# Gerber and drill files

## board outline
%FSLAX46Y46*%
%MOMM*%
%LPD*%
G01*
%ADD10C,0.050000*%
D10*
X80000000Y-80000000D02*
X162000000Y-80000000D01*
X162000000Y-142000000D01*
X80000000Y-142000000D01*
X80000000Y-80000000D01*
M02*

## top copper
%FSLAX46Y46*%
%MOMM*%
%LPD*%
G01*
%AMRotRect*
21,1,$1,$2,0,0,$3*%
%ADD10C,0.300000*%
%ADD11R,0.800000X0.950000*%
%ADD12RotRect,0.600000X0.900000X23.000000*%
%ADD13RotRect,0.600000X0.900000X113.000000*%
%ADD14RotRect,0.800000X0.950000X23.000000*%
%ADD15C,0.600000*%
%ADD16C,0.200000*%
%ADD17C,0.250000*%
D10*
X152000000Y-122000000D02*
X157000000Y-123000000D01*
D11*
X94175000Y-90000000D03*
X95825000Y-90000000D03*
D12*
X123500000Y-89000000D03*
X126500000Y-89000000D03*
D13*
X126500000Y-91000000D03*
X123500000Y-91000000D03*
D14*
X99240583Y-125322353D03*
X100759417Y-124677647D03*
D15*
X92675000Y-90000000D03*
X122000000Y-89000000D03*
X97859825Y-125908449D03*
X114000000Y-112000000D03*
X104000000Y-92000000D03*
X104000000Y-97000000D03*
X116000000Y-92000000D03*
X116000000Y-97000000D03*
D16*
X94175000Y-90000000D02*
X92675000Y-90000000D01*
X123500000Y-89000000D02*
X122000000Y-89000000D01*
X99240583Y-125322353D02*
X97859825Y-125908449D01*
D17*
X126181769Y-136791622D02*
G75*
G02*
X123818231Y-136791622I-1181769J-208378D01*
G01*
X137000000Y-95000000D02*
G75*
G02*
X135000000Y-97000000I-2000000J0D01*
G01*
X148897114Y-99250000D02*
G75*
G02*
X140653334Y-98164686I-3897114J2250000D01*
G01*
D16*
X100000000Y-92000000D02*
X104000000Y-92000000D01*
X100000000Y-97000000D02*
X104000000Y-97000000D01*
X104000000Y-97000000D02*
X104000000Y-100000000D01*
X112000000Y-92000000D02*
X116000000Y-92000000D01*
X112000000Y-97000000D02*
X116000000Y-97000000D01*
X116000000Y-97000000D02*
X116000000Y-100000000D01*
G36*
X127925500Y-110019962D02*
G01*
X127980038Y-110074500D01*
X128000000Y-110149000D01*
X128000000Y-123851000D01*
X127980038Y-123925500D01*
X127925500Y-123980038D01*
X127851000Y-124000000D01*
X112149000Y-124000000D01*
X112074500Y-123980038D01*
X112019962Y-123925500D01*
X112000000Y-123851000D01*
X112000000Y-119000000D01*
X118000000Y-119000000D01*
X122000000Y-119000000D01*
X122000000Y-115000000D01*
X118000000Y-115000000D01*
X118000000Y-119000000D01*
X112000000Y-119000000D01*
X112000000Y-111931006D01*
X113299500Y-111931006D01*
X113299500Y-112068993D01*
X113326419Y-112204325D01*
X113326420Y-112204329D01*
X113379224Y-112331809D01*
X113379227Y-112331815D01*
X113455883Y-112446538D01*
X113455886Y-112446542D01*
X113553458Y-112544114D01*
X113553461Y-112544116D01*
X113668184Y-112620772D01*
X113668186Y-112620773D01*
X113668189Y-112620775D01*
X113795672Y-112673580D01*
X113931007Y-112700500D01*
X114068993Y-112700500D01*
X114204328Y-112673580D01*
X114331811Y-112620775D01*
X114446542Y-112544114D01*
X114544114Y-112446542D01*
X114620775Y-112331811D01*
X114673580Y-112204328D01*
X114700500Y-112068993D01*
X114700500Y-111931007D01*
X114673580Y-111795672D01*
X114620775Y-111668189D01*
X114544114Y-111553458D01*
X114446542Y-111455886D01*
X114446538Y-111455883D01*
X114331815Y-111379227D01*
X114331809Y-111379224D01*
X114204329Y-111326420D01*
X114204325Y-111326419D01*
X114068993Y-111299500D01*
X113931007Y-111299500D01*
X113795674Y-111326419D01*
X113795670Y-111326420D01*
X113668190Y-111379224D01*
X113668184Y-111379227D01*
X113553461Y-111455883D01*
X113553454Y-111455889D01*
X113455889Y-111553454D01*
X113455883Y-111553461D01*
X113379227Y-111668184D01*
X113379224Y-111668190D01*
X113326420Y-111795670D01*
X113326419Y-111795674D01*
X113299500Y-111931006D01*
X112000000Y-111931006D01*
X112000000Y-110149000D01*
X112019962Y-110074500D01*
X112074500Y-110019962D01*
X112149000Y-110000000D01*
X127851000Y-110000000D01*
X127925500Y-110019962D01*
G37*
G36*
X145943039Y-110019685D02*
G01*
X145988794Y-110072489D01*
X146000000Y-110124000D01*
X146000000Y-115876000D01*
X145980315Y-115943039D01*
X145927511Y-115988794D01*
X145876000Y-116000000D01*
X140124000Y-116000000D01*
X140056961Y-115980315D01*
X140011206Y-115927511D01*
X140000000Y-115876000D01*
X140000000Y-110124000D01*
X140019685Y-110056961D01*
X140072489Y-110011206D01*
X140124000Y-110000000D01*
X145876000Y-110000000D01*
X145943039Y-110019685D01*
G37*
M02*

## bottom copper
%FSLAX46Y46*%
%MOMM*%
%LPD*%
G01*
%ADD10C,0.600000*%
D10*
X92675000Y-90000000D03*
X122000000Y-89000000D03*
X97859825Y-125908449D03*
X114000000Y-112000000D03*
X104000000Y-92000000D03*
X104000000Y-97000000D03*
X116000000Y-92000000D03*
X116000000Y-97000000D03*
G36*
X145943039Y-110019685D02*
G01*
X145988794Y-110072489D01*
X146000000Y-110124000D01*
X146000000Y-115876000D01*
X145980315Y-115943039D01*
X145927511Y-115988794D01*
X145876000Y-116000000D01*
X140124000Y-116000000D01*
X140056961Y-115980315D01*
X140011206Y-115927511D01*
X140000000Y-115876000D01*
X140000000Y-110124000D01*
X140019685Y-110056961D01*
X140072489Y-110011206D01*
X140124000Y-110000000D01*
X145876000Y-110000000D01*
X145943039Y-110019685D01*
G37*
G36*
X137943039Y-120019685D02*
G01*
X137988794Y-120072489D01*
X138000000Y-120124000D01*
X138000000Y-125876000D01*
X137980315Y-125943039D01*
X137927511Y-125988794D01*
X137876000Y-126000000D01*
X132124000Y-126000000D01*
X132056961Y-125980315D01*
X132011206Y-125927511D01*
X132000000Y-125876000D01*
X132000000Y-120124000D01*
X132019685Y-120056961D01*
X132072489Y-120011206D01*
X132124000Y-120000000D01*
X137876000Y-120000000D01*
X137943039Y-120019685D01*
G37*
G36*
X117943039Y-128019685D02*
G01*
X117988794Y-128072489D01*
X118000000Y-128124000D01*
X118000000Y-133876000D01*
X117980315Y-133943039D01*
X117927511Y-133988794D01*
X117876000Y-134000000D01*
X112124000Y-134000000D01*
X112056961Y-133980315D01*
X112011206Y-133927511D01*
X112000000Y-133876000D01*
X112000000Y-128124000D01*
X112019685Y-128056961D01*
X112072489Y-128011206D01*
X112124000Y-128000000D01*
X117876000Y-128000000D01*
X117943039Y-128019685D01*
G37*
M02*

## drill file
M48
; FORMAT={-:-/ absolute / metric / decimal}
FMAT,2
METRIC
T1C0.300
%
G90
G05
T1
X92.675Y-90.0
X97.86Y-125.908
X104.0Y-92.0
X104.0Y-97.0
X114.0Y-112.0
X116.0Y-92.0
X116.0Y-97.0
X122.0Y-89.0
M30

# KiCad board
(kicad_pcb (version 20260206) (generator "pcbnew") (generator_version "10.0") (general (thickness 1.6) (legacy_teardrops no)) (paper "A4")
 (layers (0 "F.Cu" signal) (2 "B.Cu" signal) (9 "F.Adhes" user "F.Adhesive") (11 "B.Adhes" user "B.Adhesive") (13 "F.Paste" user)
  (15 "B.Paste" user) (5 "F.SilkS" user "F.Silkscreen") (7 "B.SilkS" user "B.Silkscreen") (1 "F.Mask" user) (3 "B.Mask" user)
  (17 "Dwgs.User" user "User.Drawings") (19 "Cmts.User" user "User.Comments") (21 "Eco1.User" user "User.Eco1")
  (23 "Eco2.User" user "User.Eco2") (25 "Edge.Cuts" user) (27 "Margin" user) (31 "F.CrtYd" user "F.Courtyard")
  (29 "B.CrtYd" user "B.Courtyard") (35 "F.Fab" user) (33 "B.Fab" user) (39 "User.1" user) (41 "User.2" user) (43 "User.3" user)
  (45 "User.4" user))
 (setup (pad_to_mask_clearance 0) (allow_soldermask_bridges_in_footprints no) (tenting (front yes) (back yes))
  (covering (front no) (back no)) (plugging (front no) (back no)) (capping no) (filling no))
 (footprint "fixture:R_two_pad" (layer "F.Cu") (at 95 90)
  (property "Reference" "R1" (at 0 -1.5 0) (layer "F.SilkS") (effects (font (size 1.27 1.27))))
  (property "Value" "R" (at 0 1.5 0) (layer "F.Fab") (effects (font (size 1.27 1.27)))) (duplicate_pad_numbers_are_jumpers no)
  (pad "1" smd rect (at -0.825 0) (size 0.8 0.95) (layers "F.Cu" "F.Mask" "F.Paste") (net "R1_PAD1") (thermal_bridge_angle 45))
  (pad "2" smd rect (at 0.825 0) (size 0.8 0.95) (layers "F.Cu" "F.Mask" "F.Paste") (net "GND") (thermal_bridge_angle 45)))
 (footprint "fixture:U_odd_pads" (layer "F.Cu") (at 125 90)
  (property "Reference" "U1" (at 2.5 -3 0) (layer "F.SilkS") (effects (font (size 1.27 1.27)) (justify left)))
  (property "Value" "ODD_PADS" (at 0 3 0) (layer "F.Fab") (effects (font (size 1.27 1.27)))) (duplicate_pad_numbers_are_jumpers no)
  (pad "1" smd rect (at -1.5 -1 23) (size 0.6 0.9) (layers "F.Cu" "F.Mask" "F.Paste") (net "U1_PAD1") (thermal_bridge_angle 45))
  (pad "2" smd rect (at 1.5 -1 23) (size 0.6 0.9) (layers "F.Cu" "F.Mask" "F.Paste") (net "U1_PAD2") (thermal_bridge_angle 45))
  (pad "3" smd rect (at 1.5 1 113) (size 0.6 0.9) (layers "F.Cu" "F.Mask" "F.Paste") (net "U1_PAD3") (thermal_bridge_angle 45))
  (pad "4" smd rect (at -1.5 1 113) (size 0.6 0.9) (layers "F.Cu" "F.Mask" "F.Paste") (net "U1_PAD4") (thermal_bridge_angle 45)))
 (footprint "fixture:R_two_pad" (layer "F.Cu") (at 100 125 23)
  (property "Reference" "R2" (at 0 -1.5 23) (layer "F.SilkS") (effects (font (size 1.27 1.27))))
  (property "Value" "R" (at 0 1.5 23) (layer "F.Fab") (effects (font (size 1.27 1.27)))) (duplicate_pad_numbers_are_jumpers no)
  (pad "1" smd rect (at -0.825 0 23) (size 0.8 0.95) (layers "F.Cu" "F.Mask" "F.Paste") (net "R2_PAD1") (thermal_bridge_angle 45))
  (pad "2" smd rect (at 0.825 0 23) (size 0.8 0.95) (layers "F.Cu" "F.Mask" "F.Paste") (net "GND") (thermal_bridge_angle 45)))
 (gr_line (start 152 122) (end 157 123) (stroke (width 0.3) (type default)) (layer "F.Cu") (net "COPPER_GRAPHIC"))
 (gr_rect (start 80 80) (end 162 142) (stroke (width 0.05) (type default)) (fill no) (layer "Edge.Cuts"))
 (segment (start 94.175 90) (end 92.675 90) (width 0.2) (layer "F.Cu") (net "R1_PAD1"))
 (via (at 92.675 90) (size 0.6) (drill 0.3) (layers "F.Cu" "B.Cu") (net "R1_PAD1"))
 (segment (start 123.5 89) (end 122 89) (width 0.2) (layer "F.Cu") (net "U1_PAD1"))
 (via (at 122 89) (size 0.6) (drill 0.3) (layers "F.Cu" "B.Cu") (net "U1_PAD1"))
 (segment (start 99.240583 125.322353) (end 97.859825 125.908449) (width 0.2) (layer "F.Cu") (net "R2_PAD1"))
 (via (at 97.859825 125.908449) (size 0.6) (drill 0.3) (layers "F.Cu" "B.Cu") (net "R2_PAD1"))
 (arc (start 126.181769 136.791622) (mid 125 138.2) (end 123.818231 136.791622) (width 0.25) (layer "F.Cu") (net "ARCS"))
 (arc (start 137 95) (mid 136.414214 96.414214) (end 135 97) (width 0.25) (layer "F.Cu") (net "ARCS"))
 (arc (start 148.897114 99.25) (mid 144.412632 101.461502) (end 140.653334 98.164686) (width 0.25) (layer "F.Cu") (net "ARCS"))
 (via (at 114 112) (size 0.6) (drill 0.3) (layers "F.Cu" "B.Cu") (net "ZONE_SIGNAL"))
 (segment (start 100 92) (end 104 92) (width 0.2) (layer "F.Cu") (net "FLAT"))
 (via (at 104 92) (size 0.6) (drill 0.3) (layers "F.Cu" "B.Cu") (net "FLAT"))
 (segment (start 100 97) (end 104 97) (width 0.2) (layer "F.Cu") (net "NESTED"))
 (segment (start 104 97) (end 104 100) (width 0.2) (layer "F.Cu") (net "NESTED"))
 (via (at 104 97) (size 0.6) (drill 0.3) (layers "F.Cu" "B.Cu") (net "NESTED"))
 (segment (start 112 92) (end 116 92) (width 0.2) (locked yes) (layer "F.Cu") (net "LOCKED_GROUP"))
 (via (at 116 92) (size 0.6) (drill 0.3) (layers "F.Cu" "B.Cu") (locked yes) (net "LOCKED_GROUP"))
 (segment (start 112 97) (end 116 97) (width 0.2) (layer "F.Cu") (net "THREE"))
 (segment (start 116 97) (end 116 100) (width 0.2) (layer "F.Cu") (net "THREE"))
 (via (at 116 97) (size 0.6) (drill 0.3) (layers "F.Cu" "B.Cu") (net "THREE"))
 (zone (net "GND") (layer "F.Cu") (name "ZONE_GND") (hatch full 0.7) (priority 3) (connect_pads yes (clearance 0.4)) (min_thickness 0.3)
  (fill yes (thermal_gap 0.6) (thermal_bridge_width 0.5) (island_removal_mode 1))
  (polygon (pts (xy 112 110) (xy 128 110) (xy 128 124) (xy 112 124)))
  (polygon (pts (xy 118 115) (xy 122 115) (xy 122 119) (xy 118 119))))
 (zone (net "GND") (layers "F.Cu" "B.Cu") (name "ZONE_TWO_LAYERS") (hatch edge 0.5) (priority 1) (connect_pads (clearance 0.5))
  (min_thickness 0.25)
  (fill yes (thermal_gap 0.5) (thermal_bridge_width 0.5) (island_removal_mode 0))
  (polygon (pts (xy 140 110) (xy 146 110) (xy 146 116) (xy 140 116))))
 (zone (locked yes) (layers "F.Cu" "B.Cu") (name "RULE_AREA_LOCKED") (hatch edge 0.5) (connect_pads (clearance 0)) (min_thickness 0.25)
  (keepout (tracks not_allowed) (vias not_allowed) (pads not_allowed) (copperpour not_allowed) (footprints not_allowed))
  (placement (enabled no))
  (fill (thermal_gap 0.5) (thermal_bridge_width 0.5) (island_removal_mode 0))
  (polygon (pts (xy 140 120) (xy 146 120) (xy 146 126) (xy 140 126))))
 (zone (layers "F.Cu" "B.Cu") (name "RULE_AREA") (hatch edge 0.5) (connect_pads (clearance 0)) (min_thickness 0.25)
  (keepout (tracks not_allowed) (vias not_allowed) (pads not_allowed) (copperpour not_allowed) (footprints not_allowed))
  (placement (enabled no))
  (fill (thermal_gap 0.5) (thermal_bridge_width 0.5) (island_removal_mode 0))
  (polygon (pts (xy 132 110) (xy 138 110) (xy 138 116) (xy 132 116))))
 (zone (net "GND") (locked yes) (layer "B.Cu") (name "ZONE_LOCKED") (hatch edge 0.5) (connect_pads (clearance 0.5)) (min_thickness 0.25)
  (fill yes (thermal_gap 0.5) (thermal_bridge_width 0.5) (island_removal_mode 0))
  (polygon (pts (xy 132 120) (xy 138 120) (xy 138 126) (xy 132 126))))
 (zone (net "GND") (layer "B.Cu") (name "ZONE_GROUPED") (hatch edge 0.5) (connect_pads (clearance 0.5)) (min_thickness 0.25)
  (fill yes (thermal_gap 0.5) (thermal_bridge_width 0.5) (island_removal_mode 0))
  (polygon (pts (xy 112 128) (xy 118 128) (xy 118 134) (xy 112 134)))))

